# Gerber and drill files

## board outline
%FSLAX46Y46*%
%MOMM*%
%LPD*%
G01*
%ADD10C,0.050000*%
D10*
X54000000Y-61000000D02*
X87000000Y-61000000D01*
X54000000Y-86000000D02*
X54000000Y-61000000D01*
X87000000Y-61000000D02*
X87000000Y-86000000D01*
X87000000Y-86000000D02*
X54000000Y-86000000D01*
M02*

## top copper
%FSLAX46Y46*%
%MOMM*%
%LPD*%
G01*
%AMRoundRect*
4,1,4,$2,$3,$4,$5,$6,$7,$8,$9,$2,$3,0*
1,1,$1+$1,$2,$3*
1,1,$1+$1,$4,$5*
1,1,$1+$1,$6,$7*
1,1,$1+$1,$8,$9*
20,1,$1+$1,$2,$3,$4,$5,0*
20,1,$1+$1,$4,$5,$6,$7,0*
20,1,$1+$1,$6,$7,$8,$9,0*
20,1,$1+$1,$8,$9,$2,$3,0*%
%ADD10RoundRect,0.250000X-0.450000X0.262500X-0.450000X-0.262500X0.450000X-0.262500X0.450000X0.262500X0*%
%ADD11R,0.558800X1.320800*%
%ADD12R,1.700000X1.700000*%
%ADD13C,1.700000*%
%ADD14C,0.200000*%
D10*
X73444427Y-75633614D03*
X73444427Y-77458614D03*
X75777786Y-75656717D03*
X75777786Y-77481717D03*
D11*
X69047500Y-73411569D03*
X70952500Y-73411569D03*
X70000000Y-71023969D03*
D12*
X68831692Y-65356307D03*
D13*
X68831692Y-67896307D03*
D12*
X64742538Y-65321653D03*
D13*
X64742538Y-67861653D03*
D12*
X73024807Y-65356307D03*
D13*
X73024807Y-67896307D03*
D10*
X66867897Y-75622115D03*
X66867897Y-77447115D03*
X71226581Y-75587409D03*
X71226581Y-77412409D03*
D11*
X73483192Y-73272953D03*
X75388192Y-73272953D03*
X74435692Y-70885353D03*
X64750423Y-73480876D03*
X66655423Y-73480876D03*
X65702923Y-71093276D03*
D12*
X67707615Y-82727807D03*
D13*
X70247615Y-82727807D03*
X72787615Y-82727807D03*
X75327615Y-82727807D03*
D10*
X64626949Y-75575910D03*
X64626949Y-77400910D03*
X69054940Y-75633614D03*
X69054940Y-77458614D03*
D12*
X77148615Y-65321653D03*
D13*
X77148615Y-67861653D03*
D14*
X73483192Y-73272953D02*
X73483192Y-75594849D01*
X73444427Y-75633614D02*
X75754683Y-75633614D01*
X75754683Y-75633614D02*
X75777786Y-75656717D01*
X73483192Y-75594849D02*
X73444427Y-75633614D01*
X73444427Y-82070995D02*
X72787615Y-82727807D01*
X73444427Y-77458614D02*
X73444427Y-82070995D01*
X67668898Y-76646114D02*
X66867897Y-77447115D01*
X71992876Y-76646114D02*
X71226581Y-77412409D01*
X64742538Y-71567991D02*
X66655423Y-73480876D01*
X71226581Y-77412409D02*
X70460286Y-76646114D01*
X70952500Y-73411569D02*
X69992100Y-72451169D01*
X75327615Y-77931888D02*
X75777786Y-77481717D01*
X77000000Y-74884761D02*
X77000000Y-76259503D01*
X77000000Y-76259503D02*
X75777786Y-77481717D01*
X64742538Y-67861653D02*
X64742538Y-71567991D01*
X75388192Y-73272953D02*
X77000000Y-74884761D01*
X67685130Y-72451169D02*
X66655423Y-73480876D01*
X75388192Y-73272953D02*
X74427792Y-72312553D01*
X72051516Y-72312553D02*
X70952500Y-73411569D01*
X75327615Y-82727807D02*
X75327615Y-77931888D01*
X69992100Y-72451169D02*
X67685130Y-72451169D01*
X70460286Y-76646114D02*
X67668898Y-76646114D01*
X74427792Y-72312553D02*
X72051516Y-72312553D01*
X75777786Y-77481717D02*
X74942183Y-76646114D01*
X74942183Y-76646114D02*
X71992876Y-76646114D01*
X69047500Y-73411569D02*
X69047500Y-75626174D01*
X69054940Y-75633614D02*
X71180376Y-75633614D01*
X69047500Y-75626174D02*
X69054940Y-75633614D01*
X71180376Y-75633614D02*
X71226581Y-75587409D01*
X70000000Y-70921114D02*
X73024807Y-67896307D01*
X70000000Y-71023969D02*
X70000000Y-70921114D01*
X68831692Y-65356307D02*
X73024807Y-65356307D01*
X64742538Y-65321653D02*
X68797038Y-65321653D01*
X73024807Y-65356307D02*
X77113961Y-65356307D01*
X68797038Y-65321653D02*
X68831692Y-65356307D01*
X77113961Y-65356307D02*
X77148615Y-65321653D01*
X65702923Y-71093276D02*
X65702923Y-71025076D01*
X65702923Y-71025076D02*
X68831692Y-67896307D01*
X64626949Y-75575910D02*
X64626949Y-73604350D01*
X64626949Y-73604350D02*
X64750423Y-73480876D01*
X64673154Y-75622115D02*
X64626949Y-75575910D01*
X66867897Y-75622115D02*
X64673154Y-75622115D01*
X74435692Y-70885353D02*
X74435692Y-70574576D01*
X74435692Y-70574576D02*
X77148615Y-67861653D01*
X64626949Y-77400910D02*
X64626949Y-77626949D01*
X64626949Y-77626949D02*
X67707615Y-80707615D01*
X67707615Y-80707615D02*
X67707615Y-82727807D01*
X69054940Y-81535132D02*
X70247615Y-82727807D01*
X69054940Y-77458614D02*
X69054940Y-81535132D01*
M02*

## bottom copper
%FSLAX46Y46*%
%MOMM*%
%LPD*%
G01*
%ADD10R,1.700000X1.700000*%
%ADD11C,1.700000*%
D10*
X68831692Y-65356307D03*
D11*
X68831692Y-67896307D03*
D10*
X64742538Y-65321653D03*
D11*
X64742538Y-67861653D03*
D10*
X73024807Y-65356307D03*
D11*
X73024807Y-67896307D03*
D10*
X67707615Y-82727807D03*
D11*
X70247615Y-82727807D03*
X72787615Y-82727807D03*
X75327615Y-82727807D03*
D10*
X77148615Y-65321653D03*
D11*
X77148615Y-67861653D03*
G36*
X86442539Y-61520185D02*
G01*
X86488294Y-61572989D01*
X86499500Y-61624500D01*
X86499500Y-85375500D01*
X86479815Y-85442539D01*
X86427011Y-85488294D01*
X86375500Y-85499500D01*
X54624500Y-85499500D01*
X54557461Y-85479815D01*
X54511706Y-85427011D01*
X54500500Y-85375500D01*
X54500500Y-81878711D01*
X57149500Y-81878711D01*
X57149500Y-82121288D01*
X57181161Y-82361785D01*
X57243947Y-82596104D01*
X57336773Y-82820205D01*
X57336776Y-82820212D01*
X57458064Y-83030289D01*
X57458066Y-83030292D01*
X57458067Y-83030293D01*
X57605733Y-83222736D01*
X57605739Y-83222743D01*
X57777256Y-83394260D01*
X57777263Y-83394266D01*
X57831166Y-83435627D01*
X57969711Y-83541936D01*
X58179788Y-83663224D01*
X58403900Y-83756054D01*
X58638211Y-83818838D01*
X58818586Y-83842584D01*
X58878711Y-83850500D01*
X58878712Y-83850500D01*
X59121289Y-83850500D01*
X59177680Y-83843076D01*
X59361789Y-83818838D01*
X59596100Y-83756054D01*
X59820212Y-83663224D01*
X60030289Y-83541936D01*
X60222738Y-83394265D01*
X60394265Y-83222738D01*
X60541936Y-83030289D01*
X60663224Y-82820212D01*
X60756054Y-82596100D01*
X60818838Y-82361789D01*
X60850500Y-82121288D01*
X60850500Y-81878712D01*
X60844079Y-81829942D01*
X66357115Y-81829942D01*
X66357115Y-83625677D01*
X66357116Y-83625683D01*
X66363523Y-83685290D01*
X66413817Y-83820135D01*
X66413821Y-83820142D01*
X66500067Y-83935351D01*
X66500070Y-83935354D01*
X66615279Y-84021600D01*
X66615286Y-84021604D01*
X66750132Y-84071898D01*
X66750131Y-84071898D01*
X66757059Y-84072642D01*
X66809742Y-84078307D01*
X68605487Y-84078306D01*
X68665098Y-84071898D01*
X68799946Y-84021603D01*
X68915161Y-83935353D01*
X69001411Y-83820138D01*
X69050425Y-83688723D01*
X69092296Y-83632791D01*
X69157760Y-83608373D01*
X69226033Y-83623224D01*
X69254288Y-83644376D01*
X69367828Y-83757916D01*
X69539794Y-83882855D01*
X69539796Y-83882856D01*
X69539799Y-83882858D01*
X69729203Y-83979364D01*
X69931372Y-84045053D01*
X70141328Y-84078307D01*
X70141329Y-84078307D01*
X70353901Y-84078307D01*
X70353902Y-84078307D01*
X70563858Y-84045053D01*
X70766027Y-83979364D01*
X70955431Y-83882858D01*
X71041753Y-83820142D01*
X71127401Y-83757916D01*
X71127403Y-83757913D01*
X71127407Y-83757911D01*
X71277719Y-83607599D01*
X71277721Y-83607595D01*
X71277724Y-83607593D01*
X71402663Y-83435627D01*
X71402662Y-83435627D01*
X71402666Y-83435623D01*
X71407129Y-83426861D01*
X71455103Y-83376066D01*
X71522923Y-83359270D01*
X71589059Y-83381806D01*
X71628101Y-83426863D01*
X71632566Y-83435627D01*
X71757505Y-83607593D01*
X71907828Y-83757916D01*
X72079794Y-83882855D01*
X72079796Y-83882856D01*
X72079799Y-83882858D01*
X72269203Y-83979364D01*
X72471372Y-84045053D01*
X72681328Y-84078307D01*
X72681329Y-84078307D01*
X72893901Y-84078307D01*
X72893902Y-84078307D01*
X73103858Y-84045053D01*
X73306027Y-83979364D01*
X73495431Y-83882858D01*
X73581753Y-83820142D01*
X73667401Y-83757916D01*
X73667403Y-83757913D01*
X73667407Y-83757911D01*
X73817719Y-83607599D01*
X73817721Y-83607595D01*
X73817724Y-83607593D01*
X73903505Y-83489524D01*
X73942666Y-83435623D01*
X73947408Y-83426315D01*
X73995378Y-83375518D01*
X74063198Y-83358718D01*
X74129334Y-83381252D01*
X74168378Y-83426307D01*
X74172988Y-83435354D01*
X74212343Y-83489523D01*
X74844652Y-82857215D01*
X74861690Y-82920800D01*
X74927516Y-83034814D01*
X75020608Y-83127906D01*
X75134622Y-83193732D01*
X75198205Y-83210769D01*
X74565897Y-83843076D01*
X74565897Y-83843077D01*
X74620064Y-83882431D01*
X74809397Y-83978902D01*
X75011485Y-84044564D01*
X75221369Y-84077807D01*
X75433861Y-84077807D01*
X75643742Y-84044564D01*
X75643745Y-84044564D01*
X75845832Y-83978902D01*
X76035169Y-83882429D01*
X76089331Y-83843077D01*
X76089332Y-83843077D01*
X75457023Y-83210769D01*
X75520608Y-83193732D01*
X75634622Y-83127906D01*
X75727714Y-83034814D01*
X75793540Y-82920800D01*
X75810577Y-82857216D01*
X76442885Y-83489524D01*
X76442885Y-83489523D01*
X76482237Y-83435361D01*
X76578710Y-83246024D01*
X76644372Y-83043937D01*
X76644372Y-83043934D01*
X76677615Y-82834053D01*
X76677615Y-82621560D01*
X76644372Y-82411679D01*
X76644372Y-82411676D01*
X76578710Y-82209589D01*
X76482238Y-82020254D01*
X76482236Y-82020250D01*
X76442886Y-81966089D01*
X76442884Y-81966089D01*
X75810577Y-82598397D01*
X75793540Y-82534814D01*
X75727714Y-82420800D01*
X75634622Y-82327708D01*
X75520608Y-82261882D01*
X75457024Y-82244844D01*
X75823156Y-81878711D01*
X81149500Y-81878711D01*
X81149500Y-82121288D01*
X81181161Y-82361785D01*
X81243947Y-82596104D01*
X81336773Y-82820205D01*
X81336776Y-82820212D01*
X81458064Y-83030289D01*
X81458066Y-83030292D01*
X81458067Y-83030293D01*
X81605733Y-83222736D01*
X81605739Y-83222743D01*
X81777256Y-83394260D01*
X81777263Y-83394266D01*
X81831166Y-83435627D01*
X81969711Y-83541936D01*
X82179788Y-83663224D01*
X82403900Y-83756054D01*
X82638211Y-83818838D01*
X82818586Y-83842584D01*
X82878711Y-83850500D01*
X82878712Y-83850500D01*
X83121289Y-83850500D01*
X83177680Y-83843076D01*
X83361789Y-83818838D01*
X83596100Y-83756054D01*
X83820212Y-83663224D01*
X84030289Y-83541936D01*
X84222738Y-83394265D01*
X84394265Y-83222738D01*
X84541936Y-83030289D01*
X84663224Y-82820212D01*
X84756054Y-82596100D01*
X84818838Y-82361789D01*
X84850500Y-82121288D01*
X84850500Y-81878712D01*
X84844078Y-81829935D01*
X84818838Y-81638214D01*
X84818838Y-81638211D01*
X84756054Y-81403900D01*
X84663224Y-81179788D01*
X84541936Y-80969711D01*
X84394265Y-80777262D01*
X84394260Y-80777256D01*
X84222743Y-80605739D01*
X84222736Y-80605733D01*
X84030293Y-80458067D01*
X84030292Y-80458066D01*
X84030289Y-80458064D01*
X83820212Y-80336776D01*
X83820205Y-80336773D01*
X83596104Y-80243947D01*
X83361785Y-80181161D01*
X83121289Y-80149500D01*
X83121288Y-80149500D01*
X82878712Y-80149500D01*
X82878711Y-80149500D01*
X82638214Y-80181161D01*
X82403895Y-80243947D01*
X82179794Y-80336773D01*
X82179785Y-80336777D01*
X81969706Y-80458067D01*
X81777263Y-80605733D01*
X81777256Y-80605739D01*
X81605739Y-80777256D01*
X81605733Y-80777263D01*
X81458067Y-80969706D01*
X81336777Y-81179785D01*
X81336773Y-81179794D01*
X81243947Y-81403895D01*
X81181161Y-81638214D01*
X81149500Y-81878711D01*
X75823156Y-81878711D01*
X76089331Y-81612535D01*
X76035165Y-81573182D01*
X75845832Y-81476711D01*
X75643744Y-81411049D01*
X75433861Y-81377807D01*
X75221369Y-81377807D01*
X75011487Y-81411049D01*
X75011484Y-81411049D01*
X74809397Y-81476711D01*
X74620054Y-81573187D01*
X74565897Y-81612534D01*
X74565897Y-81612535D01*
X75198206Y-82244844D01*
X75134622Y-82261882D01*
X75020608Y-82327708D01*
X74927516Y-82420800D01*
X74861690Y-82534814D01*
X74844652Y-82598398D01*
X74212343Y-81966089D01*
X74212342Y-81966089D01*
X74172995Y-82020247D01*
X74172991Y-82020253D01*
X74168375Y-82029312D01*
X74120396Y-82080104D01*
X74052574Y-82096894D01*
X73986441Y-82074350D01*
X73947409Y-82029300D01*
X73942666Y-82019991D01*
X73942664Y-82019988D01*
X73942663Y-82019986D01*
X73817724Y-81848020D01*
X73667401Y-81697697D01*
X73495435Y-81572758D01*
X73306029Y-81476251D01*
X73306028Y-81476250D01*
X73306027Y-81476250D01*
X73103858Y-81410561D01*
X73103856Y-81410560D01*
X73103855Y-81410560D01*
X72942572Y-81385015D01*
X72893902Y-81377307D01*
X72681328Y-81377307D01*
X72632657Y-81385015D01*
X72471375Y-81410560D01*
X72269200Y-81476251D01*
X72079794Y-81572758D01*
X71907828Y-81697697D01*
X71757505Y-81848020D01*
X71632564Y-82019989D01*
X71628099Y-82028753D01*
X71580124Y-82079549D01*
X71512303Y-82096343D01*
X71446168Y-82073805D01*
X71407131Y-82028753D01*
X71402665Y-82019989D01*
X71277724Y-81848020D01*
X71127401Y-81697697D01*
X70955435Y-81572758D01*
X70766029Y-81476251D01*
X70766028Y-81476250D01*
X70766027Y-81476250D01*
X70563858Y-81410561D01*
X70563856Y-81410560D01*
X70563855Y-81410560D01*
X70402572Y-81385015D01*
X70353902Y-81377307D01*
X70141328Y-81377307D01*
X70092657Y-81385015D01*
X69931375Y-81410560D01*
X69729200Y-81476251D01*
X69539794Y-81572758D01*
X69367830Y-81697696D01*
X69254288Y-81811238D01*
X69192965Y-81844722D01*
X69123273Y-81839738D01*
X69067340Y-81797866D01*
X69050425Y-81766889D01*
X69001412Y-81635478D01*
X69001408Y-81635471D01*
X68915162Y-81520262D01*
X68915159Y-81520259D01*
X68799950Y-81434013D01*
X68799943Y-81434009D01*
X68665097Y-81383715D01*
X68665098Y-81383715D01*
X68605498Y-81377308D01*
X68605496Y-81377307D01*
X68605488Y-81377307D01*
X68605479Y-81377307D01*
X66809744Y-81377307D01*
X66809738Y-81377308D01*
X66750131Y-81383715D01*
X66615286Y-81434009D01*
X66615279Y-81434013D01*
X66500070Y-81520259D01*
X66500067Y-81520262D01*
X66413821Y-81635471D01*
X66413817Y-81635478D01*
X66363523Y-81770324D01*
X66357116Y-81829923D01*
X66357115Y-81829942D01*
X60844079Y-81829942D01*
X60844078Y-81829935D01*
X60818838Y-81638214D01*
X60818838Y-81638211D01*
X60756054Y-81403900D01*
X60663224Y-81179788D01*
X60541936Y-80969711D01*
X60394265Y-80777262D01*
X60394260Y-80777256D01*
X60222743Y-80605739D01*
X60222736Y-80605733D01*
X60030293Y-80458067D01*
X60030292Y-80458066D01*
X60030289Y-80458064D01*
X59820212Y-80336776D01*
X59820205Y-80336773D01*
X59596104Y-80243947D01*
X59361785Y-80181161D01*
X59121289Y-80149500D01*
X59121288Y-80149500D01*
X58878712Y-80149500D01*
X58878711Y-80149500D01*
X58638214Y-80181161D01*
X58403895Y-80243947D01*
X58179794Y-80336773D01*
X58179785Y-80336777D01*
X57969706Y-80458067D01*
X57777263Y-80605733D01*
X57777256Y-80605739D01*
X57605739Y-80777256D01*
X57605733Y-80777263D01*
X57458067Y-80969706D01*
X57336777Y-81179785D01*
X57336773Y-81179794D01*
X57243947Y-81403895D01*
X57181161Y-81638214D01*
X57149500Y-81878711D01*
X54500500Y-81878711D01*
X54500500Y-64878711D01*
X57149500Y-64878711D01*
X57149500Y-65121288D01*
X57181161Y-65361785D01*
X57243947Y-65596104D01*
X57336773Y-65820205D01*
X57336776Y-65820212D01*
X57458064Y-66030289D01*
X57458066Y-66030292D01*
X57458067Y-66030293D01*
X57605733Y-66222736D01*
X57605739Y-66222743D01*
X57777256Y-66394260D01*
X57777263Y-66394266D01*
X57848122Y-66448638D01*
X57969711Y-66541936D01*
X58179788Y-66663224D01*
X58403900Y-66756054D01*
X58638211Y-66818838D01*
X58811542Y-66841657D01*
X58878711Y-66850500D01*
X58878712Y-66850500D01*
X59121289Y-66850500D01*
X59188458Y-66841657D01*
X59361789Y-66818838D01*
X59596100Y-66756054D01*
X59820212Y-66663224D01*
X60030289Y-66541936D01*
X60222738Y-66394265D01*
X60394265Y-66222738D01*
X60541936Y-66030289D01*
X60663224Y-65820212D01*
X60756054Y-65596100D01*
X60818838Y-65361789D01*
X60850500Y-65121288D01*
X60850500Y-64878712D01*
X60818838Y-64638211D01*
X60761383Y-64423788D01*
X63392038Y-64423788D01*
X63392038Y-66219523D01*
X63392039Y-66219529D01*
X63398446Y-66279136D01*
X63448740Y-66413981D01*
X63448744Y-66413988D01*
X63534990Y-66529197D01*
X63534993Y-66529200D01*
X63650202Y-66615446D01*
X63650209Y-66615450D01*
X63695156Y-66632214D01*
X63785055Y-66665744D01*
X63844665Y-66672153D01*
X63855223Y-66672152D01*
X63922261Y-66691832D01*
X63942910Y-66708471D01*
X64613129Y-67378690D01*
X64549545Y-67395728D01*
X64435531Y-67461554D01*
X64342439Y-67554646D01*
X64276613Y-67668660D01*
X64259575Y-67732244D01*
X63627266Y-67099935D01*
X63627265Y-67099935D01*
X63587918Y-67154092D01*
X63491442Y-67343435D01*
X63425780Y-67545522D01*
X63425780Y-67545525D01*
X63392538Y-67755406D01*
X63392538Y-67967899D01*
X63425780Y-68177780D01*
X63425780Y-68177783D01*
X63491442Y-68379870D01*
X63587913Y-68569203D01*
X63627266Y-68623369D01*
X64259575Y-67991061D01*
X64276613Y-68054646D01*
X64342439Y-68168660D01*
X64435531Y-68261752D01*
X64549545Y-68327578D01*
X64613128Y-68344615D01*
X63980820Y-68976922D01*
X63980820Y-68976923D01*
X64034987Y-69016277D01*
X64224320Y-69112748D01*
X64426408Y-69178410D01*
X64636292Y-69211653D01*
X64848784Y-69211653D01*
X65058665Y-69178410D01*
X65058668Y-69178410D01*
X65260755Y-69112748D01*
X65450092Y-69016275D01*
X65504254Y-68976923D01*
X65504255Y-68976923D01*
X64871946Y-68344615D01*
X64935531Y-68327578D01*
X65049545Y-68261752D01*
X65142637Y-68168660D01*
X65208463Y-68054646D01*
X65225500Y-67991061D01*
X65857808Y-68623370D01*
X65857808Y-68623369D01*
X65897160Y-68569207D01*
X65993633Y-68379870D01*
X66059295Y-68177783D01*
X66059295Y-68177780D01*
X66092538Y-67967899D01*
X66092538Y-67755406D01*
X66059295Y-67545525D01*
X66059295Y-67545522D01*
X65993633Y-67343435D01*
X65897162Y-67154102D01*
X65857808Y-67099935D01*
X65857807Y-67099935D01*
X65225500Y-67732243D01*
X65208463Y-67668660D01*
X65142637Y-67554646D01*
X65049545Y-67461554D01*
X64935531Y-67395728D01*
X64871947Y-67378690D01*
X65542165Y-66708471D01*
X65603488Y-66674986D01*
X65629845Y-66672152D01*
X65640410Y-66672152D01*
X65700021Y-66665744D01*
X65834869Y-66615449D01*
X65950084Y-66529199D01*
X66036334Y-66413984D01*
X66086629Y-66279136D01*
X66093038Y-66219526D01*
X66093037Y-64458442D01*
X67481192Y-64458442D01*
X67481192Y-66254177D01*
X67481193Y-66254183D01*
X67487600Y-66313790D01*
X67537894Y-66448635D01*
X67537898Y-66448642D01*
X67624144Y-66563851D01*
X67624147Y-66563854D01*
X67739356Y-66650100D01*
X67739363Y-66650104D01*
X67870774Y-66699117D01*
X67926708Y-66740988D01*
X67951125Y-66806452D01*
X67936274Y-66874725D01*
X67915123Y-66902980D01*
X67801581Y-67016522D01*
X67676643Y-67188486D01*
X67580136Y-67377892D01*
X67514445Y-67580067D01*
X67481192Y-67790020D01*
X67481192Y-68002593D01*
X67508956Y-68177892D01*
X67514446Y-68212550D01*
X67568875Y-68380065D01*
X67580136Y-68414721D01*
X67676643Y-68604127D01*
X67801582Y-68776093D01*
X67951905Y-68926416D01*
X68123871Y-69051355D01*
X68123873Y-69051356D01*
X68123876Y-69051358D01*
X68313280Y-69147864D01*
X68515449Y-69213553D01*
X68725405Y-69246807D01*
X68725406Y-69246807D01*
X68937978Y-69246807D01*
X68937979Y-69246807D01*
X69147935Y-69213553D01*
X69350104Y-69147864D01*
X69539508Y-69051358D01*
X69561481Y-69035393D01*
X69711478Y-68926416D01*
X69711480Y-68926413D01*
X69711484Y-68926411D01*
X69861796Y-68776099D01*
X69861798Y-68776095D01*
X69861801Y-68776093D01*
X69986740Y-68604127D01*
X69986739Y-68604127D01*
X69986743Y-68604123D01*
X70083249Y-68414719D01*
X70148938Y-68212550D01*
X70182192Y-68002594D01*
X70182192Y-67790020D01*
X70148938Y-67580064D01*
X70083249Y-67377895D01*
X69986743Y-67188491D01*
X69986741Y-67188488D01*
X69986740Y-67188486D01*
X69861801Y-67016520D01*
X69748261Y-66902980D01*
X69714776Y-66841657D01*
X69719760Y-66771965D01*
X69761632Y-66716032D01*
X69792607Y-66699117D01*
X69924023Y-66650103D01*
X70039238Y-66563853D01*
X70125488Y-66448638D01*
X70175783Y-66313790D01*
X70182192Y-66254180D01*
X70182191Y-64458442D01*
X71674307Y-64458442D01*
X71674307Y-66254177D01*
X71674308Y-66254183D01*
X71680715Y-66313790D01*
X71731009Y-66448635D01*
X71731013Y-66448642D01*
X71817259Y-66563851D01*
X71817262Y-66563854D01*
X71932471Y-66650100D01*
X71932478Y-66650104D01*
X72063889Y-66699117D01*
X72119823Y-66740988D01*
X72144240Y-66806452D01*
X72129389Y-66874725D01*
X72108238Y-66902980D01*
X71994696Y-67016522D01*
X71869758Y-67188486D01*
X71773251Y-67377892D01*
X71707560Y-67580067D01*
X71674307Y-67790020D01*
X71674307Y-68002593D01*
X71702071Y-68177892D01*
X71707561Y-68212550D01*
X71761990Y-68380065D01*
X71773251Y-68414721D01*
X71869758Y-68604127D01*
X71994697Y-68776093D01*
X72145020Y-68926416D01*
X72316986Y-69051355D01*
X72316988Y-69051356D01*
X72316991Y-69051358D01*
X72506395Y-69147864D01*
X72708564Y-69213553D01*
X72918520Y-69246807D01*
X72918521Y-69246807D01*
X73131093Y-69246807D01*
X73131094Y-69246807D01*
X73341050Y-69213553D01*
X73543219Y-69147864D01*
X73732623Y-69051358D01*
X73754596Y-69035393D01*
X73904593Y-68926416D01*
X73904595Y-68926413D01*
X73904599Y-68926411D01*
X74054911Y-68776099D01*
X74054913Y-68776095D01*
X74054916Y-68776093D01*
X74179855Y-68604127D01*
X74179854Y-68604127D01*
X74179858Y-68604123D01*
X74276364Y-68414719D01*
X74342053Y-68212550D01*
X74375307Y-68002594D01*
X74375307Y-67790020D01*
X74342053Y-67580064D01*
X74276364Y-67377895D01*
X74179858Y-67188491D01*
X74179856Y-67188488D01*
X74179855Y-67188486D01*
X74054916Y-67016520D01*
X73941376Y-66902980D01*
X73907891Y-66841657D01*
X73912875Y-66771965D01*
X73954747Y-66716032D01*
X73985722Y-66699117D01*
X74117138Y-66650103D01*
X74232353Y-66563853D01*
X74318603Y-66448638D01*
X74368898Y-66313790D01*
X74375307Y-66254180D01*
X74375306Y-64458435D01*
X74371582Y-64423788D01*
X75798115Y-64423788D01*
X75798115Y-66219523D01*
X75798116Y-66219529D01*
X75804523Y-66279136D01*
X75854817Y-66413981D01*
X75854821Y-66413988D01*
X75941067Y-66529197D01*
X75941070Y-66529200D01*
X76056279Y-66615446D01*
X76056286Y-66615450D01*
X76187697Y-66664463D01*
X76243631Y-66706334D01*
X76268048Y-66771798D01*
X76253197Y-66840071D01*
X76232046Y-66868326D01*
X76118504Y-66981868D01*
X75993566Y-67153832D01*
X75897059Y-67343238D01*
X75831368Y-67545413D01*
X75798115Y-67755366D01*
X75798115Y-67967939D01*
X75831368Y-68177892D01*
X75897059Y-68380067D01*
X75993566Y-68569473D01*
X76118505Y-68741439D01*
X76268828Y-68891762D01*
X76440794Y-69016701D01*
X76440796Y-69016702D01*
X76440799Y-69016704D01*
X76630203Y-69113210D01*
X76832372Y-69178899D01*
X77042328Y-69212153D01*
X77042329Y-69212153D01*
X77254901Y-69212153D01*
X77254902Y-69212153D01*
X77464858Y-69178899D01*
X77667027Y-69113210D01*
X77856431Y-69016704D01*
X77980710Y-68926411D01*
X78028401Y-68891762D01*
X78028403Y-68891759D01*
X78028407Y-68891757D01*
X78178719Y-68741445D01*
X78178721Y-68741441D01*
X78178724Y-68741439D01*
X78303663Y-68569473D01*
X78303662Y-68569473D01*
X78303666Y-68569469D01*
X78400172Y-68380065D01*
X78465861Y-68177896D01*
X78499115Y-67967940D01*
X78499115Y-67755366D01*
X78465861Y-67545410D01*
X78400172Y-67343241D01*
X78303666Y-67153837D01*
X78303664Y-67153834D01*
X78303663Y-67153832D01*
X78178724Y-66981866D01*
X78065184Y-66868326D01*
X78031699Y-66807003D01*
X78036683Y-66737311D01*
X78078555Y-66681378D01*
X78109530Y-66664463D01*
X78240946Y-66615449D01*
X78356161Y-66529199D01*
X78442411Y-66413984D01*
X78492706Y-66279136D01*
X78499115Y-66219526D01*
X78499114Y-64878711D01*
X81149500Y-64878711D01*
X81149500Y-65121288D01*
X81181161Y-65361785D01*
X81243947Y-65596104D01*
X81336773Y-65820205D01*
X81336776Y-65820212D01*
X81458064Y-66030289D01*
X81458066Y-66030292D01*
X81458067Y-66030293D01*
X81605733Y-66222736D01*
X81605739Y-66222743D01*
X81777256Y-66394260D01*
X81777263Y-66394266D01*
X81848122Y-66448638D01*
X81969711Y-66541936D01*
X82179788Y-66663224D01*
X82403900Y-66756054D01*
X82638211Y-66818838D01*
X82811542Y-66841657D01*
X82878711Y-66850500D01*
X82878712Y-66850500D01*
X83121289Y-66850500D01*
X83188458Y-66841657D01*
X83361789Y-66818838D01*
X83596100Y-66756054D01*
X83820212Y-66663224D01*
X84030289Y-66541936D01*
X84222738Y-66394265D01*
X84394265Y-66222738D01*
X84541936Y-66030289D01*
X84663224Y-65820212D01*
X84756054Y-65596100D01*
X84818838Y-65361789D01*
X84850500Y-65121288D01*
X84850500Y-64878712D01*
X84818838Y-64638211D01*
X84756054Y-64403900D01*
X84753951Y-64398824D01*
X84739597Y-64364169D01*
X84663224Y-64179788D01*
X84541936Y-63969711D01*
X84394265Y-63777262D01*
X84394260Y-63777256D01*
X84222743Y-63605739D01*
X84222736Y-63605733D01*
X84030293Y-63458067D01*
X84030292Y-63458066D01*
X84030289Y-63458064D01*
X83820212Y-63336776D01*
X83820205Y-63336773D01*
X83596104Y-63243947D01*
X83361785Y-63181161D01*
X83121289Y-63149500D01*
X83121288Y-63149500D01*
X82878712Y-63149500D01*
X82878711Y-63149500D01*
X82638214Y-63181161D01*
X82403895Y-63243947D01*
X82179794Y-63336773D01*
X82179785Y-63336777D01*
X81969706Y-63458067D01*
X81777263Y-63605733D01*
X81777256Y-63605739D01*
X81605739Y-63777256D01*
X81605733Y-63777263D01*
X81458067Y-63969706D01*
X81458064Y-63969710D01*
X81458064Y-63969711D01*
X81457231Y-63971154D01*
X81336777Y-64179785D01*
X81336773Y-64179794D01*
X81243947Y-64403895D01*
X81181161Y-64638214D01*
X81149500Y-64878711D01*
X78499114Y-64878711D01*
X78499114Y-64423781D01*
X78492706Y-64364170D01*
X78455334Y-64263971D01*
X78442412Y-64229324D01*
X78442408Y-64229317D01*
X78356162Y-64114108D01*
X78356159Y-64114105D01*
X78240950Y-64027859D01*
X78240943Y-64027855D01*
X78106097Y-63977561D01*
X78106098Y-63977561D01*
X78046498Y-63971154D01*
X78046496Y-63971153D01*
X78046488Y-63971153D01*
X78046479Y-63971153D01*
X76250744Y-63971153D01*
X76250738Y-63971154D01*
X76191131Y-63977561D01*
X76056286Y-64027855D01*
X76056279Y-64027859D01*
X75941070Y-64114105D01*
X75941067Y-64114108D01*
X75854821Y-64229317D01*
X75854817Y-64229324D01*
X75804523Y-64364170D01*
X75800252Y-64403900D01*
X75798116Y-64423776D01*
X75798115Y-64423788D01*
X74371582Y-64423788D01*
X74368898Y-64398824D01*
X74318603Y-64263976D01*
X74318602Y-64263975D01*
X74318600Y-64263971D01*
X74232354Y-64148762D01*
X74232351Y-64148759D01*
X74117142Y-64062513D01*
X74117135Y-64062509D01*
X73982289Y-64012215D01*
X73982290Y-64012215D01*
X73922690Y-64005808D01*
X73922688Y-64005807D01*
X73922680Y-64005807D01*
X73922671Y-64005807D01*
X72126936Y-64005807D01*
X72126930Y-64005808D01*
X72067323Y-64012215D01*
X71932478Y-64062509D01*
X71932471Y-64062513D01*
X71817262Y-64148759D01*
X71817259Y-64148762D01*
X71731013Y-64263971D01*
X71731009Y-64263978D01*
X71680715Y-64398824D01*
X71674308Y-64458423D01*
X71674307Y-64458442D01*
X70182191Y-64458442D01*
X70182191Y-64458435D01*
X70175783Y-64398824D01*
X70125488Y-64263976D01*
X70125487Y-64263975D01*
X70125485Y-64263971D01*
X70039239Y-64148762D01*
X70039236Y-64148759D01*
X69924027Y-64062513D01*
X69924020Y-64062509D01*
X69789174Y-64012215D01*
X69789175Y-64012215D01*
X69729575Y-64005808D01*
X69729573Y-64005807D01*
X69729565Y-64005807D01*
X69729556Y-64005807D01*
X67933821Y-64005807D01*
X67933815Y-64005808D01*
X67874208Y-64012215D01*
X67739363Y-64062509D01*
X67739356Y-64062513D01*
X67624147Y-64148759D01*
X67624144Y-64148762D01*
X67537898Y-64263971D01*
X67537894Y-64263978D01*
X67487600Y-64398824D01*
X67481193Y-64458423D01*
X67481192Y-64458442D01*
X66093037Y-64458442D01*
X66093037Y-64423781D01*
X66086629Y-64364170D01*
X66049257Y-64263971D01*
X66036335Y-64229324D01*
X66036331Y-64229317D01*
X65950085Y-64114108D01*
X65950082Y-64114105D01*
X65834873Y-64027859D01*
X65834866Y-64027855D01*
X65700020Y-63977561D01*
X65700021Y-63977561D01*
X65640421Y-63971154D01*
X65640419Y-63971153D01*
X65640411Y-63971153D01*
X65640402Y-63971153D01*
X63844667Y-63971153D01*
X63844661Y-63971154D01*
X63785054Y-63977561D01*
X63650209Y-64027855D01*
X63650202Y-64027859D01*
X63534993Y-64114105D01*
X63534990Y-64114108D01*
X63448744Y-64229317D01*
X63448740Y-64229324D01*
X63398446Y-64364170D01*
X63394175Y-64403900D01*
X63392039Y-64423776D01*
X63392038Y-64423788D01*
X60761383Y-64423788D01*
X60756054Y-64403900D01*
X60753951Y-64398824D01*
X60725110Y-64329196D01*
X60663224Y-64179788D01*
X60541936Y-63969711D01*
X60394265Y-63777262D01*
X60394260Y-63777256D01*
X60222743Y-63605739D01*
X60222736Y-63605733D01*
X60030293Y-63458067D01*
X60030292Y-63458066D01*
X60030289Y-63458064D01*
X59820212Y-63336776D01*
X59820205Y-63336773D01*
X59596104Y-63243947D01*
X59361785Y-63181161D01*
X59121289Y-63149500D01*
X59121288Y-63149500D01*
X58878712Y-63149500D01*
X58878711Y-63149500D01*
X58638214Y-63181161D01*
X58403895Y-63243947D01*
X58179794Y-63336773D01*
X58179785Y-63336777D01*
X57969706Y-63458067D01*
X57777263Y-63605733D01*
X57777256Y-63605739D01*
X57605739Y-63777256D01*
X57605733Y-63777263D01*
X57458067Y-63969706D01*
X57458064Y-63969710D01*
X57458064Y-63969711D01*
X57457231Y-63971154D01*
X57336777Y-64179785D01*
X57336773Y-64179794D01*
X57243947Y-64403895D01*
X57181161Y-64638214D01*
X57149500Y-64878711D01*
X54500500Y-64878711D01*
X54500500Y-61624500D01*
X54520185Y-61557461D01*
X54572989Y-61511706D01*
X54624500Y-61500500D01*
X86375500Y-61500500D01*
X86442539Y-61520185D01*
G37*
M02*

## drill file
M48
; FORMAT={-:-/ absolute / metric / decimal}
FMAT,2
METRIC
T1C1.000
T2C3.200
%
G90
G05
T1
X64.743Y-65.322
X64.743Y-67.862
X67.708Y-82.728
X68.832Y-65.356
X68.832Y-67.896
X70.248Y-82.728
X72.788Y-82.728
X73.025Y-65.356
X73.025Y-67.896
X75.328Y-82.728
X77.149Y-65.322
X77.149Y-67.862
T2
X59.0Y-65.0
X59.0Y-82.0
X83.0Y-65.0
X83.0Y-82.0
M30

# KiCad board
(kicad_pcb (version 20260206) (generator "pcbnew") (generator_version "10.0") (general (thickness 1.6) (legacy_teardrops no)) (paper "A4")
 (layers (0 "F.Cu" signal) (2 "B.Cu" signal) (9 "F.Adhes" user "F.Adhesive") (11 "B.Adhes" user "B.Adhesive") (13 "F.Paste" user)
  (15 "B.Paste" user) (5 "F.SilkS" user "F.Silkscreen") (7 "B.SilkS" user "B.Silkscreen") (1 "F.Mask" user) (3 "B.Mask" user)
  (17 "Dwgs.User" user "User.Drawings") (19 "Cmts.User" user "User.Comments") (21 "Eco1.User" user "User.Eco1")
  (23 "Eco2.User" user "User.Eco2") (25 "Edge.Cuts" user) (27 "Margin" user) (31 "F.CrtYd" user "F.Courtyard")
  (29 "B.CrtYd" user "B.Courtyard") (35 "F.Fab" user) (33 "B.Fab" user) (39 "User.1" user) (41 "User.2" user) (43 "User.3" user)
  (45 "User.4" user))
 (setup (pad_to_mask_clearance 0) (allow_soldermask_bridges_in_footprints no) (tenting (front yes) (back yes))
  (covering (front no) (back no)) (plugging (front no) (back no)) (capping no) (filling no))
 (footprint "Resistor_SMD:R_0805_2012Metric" (layer "F.Cu") (at 73.444427 76.546114 -90)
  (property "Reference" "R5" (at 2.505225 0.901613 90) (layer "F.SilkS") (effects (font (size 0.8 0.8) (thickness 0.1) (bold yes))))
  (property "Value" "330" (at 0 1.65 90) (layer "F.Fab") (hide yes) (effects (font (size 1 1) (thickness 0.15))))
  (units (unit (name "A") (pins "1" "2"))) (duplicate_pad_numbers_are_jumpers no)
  (pad "1" smd roundrect (at -0.9125 0 270) (size 1.025 1.4) (layers "F.Cu" "F.Mask" "F.Paste") (roundrect_rratio 0.243902)
   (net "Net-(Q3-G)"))
  (pad "2" smd roundrect (at 0.9125 0 270) (size 1.025 1.4) (layers "F.Cu" "F.Mask" "F.Paste") (roundrect_rratio 0.243902) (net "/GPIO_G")))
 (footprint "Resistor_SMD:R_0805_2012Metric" (layer "F.Cu") (at 75.777786 76.569217 -90)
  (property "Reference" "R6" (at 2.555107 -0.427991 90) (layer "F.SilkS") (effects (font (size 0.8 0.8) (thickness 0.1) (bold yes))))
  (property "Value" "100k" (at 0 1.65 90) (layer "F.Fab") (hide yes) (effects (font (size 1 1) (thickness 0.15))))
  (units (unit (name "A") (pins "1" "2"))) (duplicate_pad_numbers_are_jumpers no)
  (pad "1" smd roundrect (at -0.9125 0 270) (size 1.025 1.4) (layers "F.Cu" "F.Mask" "F.Paste") (roundrect_rratio 0.243902)
   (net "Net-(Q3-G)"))
  (pad "2" smd roundrect (at 0.9125 0 270) (size 1.025 1.4) (layers "F.Cu" "F.Mask" "F.Paste") (roundrect_rratio 0.243902) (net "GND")))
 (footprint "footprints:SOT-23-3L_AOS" (layer "F.Cu") (at 70 72.217769)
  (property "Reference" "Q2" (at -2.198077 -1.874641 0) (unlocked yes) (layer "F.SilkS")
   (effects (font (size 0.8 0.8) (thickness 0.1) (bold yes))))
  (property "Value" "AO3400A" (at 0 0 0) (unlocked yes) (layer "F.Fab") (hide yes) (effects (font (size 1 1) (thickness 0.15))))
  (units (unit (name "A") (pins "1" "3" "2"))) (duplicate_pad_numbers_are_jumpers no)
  (pad "1" smd rect (at -0.9525 1.1938) (size 0.5588 1.3208) (layers "F.Cu" "F.Mask" "F.Paste") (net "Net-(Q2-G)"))
  (pad "2" smd rect (at 0.9525 1.1938) (size 0.5588 1.3208) (layers "F.Cu" "F.Mask" "F.Paste") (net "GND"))
  (pad "3" smd rect (at 0 -1.1938) (size 0.5588 1.3208) (layers "F.Cu" "F.Mask" "F.Paste") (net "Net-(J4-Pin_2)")))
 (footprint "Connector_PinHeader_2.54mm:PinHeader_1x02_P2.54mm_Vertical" (layer "F.Cu") (at 68.831692 65.356307)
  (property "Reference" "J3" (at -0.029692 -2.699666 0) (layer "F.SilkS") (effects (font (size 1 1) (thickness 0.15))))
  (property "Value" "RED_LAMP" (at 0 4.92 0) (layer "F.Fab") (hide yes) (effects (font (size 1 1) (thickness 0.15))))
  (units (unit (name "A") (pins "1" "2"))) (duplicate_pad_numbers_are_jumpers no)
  (pad "1" thru_hole rect (at 0 0) (size 1.7 1.7) (drill 1) (layers "*.Cu" "*.Mask") (remove_unused_layers no) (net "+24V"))
  (pad "2" thru_hole circle (at 0 2.54) (size 1.7 1.7) (drill 1) (layers "*.Cu" "*.Mask") (remove_unused_layers no) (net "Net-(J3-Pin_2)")))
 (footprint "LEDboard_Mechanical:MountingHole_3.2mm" (layer "F.Cu") (at 59 65)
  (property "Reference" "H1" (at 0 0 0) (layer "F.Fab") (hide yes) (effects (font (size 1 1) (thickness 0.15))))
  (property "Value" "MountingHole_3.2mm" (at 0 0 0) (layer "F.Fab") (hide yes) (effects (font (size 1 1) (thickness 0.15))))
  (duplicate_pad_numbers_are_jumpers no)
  (pad "" np_thru_hole circle (at 0 0) (size 3.2 3.2) (drill 3.2) (layers "*.Cu" "*.Mask")))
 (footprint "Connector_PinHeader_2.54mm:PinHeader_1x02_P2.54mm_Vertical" (layer "F.Cu") (at 64.742538 65.321653)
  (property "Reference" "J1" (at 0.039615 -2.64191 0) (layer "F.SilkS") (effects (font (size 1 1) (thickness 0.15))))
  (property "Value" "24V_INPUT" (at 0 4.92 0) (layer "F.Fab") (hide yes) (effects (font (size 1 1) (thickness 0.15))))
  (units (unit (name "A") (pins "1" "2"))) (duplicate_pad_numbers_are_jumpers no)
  (pad "1" thru_hole rect (at 0 0) (size 1.7 1.7) (drill 1) (layers "*.Cu" "*.Mask") (remove_unused_layers no) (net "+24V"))
  (pad "2" thru_hole circle (at 0 2.54) (size 1.7 1.7) (drill 1) (layers "*.Cu" "*.Mask") (remove_unused_layers no) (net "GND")))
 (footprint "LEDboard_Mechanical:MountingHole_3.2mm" (layer "F.Cu") (at 59 82)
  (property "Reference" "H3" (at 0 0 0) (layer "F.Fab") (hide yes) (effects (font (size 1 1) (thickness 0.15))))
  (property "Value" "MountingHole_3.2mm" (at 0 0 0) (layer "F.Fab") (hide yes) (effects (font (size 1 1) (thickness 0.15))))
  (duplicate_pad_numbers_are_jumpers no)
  (pad "" np_thru_hole circle (at 0 0) (size 3.2 3.2) (drill 3.2) (layers "*.Cu" "*.Mask")))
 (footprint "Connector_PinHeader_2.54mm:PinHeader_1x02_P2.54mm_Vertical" (layer "F.Cu") (at 73.024807 65.356307)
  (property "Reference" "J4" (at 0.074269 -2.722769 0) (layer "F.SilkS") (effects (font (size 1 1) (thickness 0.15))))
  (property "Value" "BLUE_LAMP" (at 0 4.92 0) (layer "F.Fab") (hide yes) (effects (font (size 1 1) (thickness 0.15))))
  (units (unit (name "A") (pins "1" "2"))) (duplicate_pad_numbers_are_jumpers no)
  (pad "1" thru_hole rect (at 0 0) (size 1.7 1.7) (drill 1) (layers "*.Cu" "*.Mask") (remove_unused_layers no) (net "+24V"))
  (pad "2" thru_hole circle (at 0 2.54) (size 1.7 1.7) (drill 1) (layers "*.Cu" "*.Mask") (remove_unused_layers no) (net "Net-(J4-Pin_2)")))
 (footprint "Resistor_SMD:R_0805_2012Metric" (layer "F.Cu") (at 66.867897 76.534615 -90)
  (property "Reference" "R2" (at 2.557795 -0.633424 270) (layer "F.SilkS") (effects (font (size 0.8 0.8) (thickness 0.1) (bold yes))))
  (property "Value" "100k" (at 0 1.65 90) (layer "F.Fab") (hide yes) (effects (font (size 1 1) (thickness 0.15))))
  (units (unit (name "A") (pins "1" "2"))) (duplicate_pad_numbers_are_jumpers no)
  (pad "1" smd roundrect (at -0.9125 0 270) (size 1.025 1.4) (layers "F.Cu" "F.Mask" "F.Paste") (roundrect_rratio 0.243902)
   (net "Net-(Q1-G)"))
  (pad "2" smd roundrect (at 0.9125 0 270) (size 1.025 1.4) (layers "F.Cu" "F.Mask" "F.Paste") (roundrect_rratio 0.243902) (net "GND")))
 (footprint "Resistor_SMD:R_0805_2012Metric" (layer "F.Cu") (at 71.226581 76.499909 -90)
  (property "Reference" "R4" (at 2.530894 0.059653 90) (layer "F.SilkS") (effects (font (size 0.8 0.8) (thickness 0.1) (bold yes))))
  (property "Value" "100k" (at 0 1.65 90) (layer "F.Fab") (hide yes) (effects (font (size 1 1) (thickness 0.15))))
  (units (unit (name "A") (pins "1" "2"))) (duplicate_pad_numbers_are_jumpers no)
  (pad "1" smd roundrect (at -0.9125 0 270) (size 1.025 1.4) (layers "F.Cu" "F.Mask" "F.Paste") (roundrect_rratio 0.243902)
   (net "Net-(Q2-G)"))
  (pad "2" smd roundrect (at 0.9125 0 270) (size 1.025 1.4) (layers "F.Cu" "F.Mask" "F.Paste") (roundrect_rratio 0.243902) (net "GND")))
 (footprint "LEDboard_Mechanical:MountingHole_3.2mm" (layer "F.Cu") (at 83 65)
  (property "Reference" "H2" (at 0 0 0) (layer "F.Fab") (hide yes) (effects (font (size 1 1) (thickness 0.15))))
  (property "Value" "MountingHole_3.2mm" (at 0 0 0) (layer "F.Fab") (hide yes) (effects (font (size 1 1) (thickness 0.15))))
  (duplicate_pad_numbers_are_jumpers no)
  (pad "" np_thru_hole circle (at 0 0) (size 3.2 3.2) (drill 3.2) (layers "*.Cu" "*.Mask")))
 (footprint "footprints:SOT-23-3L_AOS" (layer "F.Cu") (at 74.435692 72.079153)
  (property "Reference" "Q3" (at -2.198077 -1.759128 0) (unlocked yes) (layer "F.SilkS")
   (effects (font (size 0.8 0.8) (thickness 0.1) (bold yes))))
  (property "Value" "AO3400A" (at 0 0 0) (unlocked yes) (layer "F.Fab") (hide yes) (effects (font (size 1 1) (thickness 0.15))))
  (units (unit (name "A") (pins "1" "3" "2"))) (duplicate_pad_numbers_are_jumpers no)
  (pad "1" smd rect (at -0.9525 1.1938) (size 0.5588 1.3208) (layers "F.Cu" "F.Mask" "F.Paste") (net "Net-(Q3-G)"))
  (pad "2" smd rect (at 0.9525 1.1938) (size 0.5588 1.3208) (layers "F.Cu" "F.Mask" "F.Paste") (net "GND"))
  (pad "3" smd rect (at 0 -1.1938) (size 0.5588 1.3208) (layers "F.Cu" "F.Mask" "F.Paste") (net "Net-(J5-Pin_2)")))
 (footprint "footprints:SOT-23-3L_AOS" (layer "F.Cu") (at 65.702923 72.287076)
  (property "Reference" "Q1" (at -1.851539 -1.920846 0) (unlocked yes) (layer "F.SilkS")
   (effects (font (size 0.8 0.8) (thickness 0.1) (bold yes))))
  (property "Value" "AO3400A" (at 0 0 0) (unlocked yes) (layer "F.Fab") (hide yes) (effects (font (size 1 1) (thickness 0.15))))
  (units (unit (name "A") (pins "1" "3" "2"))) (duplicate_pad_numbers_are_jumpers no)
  (pad "1" smd rect (at -0.9525 1.1938) (size 0.5588 1.3208) (layers "F.Cu" "F.Mask" "F.Paste") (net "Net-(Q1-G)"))
  (pad "2" smd rect (at 0.9525 1.1938) (size 0.5588 1.3208) (layers "F.Cu" "F.Mask" "F.Paste") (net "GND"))
  (pad "3" smd rect (at 0 -1.1938) (size 0.5588 1.3208) (layers "F.Cu" "F.Mask" "F.Paste") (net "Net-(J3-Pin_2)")))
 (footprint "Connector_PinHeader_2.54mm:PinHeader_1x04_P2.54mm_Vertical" (layer "F.Cu") (at 67.707615 82.727807 90)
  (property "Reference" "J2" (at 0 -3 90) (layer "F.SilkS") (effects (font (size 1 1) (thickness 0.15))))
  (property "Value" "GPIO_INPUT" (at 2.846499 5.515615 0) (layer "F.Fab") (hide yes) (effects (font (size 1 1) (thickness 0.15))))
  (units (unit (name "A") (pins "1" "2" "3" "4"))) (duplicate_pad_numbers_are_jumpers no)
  (pad "1" thru_hole rect (at 0 0 90) (size 1.7 1.7) (drill 1) (layers "*.Cu" "*.Mask") (remove_unused_layers no) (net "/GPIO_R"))
  (pad "2" thru_hole circle (at 0 2.54 90) (size 1.7 1.7) (drill 1) (layers "*.Cu" "*.Mask") (remove_unused_layers no) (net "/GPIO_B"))
  (pad "3" thru_hole circle (at 0 5.08 90) (size 1.7 1.7) (drill 1) (layers "*.Cu" "*.Mask") (remove_unused_layers no) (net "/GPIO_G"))
  (pad "4" thru_hole circle (at 0 7.62 90) (size 1.7 1.7) (drill 1) (layers "*.Cu" "*.Mask") (remove_unused_layers no) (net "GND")))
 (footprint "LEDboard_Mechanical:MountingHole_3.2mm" (layer "F.Cu") (at 83 82)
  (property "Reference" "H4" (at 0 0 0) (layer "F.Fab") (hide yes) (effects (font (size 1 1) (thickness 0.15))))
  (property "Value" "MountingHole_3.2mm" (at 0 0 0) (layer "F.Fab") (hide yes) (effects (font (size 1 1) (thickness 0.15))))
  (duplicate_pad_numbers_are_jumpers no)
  (pad "" np_thru_hole circle (at 0 0) (size 3.2 3.2) (drill 3.2) (layers "*.Cu" "*.Mask")))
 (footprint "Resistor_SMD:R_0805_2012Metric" (layer "F.Cu") (at 64.626949 76.48841 -90)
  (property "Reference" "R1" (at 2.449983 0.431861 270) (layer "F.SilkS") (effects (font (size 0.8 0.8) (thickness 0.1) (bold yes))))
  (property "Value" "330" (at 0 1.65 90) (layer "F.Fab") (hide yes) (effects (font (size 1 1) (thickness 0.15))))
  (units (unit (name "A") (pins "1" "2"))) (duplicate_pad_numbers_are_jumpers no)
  (pad "1" smd roundrect (at -0.9125 0 270) (size 1.025 1.4) (layers "F.Cu" "F.Mask" "F.Paste") (roundrect_rratio 0.243902)
   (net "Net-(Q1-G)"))
  (pad "2" smd roundrect (at 0.9125 0 270) (size 1.025 1.4) (layers "F.Cu" "F.Mask" "F.Paste") (roundrect_rratio 0.243902) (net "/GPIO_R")))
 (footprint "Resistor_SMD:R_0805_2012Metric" (layer "F.Cu") (at 69.05494 76.546114 -90)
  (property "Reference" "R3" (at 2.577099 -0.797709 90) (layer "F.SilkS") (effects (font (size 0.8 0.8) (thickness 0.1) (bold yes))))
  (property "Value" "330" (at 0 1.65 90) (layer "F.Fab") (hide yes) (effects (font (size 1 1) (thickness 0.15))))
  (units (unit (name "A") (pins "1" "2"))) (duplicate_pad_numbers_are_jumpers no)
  (pad "1" smd roundrect (at -0.9125 0 270) (size 1.025 1.4) (layers "F.Cu" "F.Mask" "F.Paste") (roundrect_rratio 0.243902)
   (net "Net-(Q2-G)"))
  (pad "2" smd roundrect (at 0.9125 0 270) (size 1.025 1.4) (layers "F.Cu" "F.Mask" "F.Paste") (roundrect_rratio 0.243902) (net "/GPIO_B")))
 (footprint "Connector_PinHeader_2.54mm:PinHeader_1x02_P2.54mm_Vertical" (layer "F.Cu") (at 77.148615 65.321653)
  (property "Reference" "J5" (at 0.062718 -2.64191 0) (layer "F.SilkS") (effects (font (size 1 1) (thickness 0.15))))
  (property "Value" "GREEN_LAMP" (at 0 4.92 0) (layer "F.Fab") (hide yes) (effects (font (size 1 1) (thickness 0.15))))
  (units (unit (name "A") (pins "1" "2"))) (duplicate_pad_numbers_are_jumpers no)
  (pad "1" thru_hole rect (at 0 0) (size 1.7 1.7) (drill 1) (layers "*.Cu" "*.Mask") (remove_unused_layers no) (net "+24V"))
  (pad "2" thru_hole circle (at 0 2.54) (size 1.7 1.7) (drill 1) (layers "*.Cu" "*.Mask") (remove_unused_layers no) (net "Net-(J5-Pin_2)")))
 (gr_line (start 54 61) (end 87 61) (stroke (width 0.05) (type default)) (layer "Edge.Cuts"))
 (gr_line (start 54 86) (end 54 61) (stroke (width 0.05) (type default)) (layer "Edge.Cuts"))
 (gr_line (start 87 61) (end 87 86) (stroke (width 0.05) (type default)) (layer "Edge.Cuts"))
 (gr_line (start 87 86) (end 54 86) (stroke (width 0.05) (type default)) (layer "Edge.Cuts"))
 (segment (start 73.483192 73.272953) (end 73.483192 75.594849) (width 0.2) (layer "F.Cu") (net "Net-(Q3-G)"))
 (segment (start 73.444427 75.633614) (end 75.754683 75.633614) (width 0.2) (layer "F.Cu") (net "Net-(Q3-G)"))
 (segment (start 75.754683 75.633614) (end 75.777786 75.656717) (width 0.2) (layer "F.Cu") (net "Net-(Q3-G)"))
 (segment (start 73.483192 75.594849) (end 73.444427 75.633614) (width 0.2) (layer "F.Cu") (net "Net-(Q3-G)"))
 (segment (start 73.444427 82.070995) (end 72.787615 82.727807) (width 0.2) (layer "F.Cu") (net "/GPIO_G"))
 (segment (start 73.444427 77.458614) (end 73.444427 82.070995) (width 0.2) (layer "F.Cu") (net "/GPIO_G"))
 (segment (start 67.668898 76.646114) (end 66.867897 77.447115) (width 0.2) (layer "F.Cu") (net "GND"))
 (segment (start 71.992876 76.646114) (end 71.226581 77.412409) (width 0.2) (layer "F.Cu") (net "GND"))
 (segment (start 64.742538 71.567991) (end 66.655423 73.480876) (width 0.2) (layer "F.Cu") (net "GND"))
 (segment (start 71.226581 77.412409) (end 70.460286 76.646114) (width 0.2) (layer "F.Cu") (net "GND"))
 (segment (start 70.9525 73.411569) (end 69.9921 72.451169) (width 0.2) (layer "F.Cu") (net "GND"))
 (segment (start 75.327615 77.931888) (end 75.777786 77.481717) (width 0.2) (layer "F.Cu") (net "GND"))
 (segment (start 77 74.884761) (end 77 76.259503) (width 0.2) (layer "F.Cu") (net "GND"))
 (segment (start 77 76.259503) (end 75.777786 77.481717) (width 0.2) (layer "F.Cu") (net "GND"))
 (segment (start 64.742538 67.861653) (end 64.742538 71.567991) (width 0.2) (layer "F.Cu") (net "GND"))
 (segment (start 75.388192 73.272953) (end 77 74.884761) (width 0.2) (layer "F.Cu") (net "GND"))
 (segment (start 67.68513 72.451169) (end 66.655423 73.480876) (width 0.2) (layer "F.Cu") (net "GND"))
 (segment (start 75.388192 73.272953) (end 74.427792 72.312553) (width 0.2) (layer "F.Cu") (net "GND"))
 (segment (start 72.051516 72.312553) (end 70.9525 73.411569) (width 0.2) (layer "F.Cu") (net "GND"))
 (segment (start 75.327615 82.727807) (end 75.327615 77.931888) (width 0.2) (layer "F.Cu") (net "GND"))
 (segment (start 69.9921 72.451169) (end 67.68513 72.451169) (width 0.2) (layer "F.Cu") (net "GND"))
 (segment (start 70.460286 76.646114) (end 67.668898 76.646114) (width 0.2) (layer "F.Cu") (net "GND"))
 (segment (start 74.427792 72.312553) (end 72.051516 72.312553) (width 0.2) (layer "F.Cu") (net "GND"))
 (segment (start 75.777786 77.481717) (end 74.942183 76.646114) (width 0.2) (layer "F.Cu") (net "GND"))
 (segment (start 74.942183 76.646114) (end 71.992876 76.646114) (width 0.2) (layer "F.Cu") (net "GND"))
 (segment (start 69.0475 73.411569) (end 69.0475 75.626174) (width 0.2) (layer "F.Cu") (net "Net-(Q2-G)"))
 (segment (start 69.05494 75.633614) (end 71.180376 75.633614) (width 0.2) (layer "F.Cu") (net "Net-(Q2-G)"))
 (segment (start 69.0475 75.626174) (end 69.05494 75.633614) (width 0.2) (layer "F.Cu") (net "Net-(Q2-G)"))
 (segment (start 71.180376 75.633614) (end 71.226581 75.587409) (width 0.2) (layer "F.Cu") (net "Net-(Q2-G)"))
 (segment (start 70 70.921114) (end 73.024807 67.896307) (width 0.2) (layer "F.Cu") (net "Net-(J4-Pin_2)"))
 (segment (start 70 71.023969) (end 70 70.921114) (width 0.2) (layer "F.Cu") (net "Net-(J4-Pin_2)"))
 (segment (start 68.831692 65.356307) (end 73.024807 65.356307) (width 0.2) (layer "F.Cu") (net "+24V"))
 (segment (start 64.742538 65.321653) (end 68.797038 65.321653) (width 0.2) (layer "F.Cu") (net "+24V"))
 (segment (start 73.024807 65.356307) (end 77.113961 65.356307) (width 0.2) (layer "F.Cu") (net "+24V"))
 (segment (start 68.797038 65.321653) (end 68.831692 65.356307) (width 0.2) (layer "F.Cu") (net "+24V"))
 (segment (start 77.113961 65.356307) (end 77.148615 65.321653) (width 0.2) (layer "F.Cu") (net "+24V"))
 (segment (start 65.702923 71.093276) (end 65.702923 71.025076) (width 0.2) (layer "F.Cu") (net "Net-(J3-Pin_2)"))
 (segment (start 65.702923 71.025076) (end 68.831692 67.896307) (width 0.2) (layer "F.Cu") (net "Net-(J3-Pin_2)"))
 (segment (start 64.626949 75.57591) (end 64.626949 73.60435) (width 0.2) (layer "F.Cu") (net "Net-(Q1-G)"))
 (segment (start 64.626949 73.60435) (end 64.750423 73.480876) (width 0.2) (layer "F.Cu") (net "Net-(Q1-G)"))
 (segment (start 64.673154 75.622115) (end 64.626949 75.57591) (width 0.2) (layer "F.Cu") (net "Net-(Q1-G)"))
 (segment (start 66.867897 75.622115) (end 64.673154 75.622115) (width 0.2) (layer "F.Cu") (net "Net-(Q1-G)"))
 (segment (start 74.435692 70.885353) (end 74.435692 70.574576) (width 0.2) (layer "F.Cu") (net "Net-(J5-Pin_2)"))
 (segment (start 74.435692 70.574576) (end 77.148615 67.861653) (width 0.2) (layer "F.Cu") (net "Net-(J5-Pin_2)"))
 (segment (start 64.626949 77.40091) (end 64.626949 77.626949) (width 0.2) (layer "F.Cu") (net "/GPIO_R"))
 (segment (start 64.626949 77.626949) (end 67.707615 80.707615) (width 0.2) (layer "F.Cu") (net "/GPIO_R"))
 (segment (start 67.707615 80.707615) (end 67.707615 82.727807) (width 0.2) (layer "F.Cu") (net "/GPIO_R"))
 (segment (start 69.05494 81.535132) (end 70.247615 82.727807) (width 0.2) (layer "F.Cu") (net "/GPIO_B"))
 (segment (start 69.05494 77.458614) (end 69.05494 81.535132) (width 0.2) (layer "F.Cu") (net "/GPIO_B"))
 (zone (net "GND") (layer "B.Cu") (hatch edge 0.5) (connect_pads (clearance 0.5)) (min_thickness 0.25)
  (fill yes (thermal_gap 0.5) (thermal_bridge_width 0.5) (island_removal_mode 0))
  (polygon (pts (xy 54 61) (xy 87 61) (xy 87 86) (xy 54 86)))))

